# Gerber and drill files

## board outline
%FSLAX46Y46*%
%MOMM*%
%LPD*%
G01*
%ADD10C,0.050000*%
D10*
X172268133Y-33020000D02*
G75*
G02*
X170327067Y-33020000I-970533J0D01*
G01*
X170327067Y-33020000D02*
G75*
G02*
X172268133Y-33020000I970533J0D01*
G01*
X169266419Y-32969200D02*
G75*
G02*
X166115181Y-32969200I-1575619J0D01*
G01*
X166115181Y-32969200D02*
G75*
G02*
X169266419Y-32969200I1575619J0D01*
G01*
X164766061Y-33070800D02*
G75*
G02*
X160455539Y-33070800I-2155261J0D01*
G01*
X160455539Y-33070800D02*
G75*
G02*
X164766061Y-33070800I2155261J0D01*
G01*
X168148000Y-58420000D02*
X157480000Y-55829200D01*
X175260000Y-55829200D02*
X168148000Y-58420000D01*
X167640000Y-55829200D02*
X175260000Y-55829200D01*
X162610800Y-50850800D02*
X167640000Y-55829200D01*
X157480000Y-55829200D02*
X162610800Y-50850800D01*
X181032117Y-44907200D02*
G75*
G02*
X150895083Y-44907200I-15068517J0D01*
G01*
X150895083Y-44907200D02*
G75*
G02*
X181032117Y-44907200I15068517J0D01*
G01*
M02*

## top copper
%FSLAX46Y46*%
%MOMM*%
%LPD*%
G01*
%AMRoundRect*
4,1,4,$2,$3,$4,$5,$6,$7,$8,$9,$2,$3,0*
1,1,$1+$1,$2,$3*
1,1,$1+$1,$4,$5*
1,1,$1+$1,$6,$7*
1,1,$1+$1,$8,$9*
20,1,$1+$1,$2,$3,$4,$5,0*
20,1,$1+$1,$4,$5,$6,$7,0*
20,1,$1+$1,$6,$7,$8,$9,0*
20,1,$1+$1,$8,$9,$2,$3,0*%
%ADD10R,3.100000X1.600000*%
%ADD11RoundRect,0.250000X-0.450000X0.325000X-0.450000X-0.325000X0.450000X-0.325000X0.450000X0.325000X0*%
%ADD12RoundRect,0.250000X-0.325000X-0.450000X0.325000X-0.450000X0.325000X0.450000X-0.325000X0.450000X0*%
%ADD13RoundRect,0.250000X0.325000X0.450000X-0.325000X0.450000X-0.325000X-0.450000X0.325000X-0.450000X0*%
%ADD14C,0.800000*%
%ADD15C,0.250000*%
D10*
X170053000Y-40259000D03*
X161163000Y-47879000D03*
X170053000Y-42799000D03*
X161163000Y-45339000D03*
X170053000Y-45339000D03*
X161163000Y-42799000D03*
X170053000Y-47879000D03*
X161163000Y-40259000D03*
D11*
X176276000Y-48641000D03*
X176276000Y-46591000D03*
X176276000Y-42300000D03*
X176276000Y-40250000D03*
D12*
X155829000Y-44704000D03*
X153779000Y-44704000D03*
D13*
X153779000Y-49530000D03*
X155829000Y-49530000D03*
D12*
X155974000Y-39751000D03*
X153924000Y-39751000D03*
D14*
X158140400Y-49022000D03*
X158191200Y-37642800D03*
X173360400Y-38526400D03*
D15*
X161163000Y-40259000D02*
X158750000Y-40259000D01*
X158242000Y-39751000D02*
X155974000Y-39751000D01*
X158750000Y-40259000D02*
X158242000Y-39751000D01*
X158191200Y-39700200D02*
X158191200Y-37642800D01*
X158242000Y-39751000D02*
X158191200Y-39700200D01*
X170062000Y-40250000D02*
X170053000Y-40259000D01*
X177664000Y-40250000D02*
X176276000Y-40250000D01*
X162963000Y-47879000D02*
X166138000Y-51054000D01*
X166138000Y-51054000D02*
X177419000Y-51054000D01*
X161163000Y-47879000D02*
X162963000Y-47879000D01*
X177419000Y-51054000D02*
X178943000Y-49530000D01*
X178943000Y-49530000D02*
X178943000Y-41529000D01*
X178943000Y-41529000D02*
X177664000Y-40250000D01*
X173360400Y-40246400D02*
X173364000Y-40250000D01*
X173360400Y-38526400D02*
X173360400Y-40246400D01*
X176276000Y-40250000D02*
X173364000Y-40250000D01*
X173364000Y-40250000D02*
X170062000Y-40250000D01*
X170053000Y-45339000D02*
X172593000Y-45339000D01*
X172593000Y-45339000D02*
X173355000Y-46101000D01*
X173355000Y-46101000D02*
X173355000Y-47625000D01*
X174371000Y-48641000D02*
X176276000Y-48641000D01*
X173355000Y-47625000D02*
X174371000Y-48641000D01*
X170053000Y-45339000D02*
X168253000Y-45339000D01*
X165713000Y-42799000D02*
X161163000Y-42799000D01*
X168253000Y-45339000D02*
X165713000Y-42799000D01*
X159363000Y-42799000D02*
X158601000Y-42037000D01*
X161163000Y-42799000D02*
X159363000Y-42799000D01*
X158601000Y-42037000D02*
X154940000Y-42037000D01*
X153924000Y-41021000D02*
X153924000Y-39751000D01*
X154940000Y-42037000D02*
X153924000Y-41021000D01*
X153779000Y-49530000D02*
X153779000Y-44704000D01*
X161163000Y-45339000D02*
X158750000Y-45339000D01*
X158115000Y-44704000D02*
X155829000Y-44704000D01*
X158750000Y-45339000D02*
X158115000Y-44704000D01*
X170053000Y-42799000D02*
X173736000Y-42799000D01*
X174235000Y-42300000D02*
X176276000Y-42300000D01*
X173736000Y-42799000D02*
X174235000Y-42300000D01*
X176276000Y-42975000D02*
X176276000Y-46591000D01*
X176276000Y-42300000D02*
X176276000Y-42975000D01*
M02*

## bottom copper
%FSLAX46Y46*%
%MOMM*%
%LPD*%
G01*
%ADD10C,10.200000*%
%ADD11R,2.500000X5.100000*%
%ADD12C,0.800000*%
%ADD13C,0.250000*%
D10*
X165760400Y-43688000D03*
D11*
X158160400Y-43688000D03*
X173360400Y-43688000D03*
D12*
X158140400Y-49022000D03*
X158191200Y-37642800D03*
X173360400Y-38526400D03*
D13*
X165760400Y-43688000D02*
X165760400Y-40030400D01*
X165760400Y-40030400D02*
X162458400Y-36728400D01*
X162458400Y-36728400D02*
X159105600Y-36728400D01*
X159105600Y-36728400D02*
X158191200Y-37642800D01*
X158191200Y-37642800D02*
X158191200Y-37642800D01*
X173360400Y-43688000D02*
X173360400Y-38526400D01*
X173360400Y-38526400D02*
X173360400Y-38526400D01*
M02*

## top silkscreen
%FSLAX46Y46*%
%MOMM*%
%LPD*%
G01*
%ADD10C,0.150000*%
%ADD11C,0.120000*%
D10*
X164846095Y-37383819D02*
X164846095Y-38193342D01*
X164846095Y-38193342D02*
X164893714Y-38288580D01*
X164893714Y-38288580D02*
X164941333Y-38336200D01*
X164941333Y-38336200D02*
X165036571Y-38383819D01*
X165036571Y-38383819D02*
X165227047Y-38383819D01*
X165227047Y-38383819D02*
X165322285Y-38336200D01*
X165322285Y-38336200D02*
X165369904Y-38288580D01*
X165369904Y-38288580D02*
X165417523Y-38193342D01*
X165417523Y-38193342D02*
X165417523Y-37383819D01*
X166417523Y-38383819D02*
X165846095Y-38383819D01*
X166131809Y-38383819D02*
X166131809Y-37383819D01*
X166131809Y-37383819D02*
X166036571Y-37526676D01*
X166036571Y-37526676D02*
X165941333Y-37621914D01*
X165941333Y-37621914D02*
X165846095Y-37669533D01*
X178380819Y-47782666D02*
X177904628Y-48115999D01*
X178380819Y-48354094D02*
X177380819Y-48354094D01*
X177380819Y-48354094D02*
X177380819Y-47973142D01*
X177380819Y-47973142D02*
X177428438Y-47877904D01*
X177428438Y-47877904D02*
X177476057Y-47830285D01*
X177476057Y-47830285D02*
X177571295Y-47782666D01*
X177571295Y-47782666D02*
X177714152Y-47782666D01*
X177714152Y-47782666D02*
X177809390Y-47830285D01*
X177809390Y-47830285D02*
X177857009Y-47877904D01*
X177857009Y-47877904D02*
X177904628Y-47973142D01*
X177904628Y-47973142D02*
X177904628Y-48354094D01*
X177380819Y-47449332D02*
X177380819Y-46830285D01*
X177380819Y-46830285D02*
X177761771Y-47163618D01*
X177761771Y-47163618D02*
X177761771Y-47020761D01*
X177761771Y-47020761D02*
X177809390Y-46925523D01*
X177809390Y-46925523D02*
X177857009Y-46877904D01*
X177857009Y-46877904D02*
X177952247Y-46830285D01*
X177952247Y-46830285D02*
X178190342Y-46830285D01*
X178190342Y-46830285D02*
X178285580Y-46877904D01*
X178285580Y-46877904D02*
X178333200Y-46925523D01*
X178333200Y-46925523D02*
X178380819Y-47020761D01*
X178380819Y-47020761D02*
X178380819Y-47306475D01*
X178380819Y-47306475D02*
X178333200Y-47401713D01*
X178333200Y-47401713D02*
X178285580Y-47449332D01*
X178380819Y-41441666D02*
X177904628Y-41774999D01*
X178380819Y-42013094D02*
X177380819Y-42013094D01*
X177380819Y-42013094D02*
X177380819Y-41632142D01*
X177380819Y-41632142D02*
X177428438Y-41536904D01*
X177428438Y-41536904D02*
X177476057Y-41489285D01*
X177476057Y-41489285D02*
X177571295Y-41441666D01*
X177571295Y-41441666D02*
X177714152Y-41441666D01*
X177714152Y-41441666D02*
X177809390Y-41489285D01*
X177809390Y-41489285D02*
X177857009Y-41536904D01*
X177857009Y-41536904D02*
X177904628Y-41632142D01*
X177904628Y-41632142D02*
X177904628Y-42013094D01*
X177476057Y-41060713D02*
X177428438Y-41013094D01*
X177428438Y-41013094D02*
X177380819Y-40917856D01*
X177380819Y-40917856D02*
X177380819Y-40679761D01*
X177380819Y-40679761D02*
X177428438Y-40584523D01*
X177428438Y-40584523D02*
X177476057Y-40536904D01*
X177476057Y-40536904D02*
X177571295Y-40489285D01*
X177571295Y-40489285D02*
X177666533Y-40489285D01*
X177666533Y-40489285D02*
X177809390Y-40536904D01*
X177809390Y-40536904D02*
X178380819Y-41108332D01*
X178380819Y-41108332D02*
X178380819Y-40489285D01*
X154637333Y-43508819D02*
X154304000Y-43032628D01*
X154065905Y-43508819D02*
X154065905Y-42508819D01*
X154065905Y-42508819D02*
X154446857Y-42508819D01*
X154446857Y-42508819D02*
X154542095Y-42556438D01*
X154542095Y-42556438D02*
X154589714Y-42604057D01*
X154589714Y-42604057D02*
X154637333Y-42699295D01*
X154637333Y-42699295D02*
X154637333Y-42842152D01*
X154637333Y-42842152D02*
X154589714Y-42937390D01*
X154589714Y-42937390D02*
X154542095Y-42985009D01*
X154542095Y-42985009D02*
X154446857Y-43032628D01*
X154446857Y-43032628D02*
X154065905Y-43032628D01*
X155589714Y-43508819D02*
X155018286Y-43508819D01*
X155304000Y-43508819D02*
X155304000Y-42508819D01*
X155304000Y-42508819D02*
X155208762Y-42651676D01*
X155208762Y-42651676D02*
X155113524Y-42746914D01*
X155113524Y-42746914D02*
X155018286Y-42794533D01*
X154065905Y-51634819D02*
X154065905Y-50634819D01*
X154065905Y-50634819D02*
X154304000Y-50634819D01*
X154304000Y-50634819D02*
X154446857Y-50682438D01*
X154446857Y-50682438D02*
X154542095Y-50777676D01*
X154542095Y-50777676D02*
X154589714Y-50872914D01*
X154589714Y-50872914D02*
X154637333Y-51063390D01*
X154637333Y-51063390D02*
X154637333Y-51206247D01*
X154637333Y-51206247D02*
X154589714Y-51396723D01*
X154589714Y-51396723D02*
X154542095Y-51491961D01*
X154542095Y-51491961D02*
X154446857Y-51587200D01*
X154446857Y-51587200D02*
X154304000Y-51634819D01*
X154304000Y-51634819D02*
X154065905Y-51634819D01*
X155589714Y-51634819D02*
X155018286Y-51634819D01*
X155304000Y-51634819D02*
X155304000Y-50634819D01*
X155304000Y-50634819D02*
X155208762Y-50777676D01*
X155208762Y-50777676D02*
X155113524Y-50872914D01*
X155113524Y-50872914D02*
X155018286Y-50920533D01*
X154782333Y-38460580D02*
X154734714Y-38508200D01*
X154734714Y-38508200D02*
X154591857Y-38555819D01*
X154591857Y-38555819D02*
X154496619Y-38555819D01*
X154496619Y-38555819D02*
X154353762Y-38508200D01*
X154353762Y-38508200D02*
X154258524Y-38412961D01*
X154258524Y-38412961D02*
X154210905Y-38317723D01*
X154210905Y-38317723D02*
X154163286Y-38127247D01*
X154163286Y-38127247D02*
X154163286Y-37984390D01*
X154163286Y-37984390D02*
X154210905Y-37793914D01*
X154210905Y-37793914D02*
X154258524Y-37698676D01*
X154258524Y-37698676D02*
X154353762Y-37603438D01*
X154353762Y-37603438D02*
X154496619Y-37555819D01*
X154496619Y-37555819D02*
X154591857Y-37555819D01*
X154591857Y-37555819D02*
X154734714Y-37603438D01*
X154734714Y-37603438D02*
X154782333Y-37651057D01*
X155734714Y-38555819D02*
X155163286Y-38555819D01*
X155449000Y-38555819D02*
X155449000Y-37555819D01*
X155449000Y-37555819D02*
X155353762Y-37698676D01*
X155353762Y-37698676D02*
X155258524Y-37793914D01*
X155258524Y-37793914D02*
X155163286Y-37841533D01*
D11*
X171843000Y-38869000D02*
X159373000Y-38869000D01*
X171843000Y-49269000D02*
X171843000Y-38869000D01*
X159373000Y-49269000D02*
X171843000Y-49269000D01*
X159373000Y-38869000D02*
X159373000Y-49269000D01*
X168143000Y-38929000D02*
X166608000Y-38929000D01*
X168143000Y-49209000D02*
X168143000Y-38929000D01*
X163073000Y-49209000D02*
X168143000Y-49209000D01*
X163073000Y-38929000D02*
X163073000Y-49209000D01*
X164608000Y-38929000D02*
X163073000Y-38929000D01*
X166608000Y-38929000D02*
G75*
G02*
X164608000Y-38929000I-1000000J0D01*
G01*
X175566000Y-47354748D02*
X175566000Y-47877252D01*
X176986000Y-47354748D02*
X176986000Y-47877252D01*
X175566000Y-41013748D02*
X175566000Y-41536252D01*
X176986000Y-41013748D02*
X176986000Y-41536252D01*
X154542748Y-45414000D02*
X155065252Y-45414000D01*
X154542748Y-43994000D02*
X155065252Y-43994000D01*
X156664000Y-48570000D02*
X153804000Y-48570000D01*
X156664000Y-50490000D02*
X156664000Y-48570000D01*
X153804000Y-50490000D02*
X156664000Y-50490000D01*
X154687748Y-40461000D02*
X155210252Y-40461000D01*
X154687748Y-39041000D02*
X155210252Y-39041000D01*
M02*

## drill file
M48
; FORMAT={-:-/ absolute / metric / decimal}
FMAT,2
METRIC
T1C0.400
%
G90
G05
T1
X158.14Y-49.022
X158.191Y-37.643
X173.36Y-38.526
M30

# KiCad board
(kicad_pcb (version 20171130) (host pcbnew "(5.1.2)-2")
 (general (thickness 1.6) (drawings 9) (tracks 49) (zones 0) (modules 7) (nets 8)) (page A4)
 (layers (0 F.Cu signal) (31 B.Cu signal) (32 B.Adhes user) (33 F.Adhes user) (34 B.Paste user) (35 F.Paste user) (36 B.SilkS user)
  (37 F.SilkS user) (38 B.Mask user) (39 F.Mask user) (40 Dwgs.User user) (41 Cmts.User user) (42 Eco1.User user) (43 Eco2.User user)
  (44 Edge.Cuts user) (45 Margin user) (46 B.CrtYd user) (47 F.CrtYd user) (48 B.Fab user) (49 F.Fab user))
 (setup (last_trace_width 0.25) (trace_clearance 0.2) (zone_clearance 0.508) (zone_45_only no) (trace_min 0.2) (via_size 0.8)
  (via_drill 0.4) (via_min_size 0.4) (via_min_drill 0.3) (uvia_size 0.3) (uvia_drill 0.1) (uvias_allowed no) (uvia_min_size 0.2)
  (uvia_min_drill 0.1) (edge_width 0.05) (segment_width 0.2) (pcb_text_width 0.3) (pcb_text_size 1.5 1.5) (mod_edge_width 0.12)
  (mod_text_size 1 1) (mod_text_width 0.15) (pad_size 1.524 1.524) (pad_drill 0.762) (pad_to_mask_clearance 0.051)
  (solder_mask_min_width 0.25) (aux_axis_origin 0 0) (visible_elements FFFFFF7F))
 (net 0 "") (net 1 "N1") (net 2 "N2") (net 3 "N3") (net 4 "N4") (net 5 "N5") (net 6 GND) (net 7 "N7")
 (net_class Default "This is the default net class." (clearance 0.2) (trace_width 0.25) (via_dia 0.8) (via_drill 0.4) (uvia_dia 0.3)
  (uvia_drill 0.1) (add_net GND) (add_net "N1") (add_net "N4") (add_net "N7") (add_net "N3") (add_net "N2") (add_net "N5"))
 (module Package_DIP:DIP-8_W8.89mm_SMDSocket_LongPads (layer F.Cu) (at 165.608 44.069)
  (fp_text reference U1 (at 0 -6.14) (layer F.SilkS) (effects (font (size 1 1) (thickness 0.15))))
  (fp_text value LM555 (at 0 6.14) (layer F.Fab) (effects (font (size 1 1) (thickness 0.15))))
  (fp_line (start 6.235 -5.2) (end -6.235 -5.2) (layer F.SilkS) (width 0.12))
  (fp_line (start 6.235 5.2) (end 6.235 -5.2) (layer F.SilkS) (width 0.12))
  (fp_line (start -6.235 5.2) (end 6.235 5.2) (layer F.SilkS) (width 0.12))
  (fp_line (start -6.235 -5.2) (end -6.235 5.2) (layer F.SilkS) (width 0.12))
  (fp_line (start 2.535 -5.14) (end 1 -5.14) (layer F.SilkS) (width 0.12))
  (fp_line (start 2.535 5.14) (end 2.535 -5.14) (layer F.SilkS) (width 0.12))
  (fp_line (start -2.535 5.14) (end 2.535 5.14) (layer F.SilkS) (width 0.12))
  (fp_line (start -2.535 -5.14) (end -2.535 5.14) (layer F.SilkS) (width 0.12))
  (fp_line (start -1 -5.14) (end -2.535 -5.14) (layer F.SilkS) (width 0.12))
  (fp_arc (start 0 -5.14) (end -1 -5.14) (angle -180) (layer F.SilkS) (width 0.12))
  (pad 8 smd rect (at 4.445 -3.81) (size 3.1 1.6) (layers F.Cu F.Paste F.Mask) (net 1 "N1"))
  (pad 4 smd rect (at -4.445 3.81) (size 3.1 1.6) (layers F.Cu F.Paste F.Mask) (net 1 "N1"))
  (pad 7 smd rect (at 4.445 -1.27) (size 3.1 1.6) (layers F.Cu F.Paste F.Mask) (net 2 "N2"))
  (pad 3 smd rect (at -4.445 1.27) (size 3.1 1.6) (layers F.Cu F.Paste F.Mask) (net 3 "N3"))
  (pad 6 smd rect (at 4.445 1.27) (size 3.1 1.6) (layers F.Cu F.Paste F.Mask) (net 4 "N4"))
  (pad 2 smd rect (at -4.445 -1.27) (size 3.1 1.6) (layers F.Cu F.Paste F.Mask) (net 4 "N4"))
  (pad 5 smd rect (at 4.445 3.81) (size 3.1 1.6) (layers F.Cu F.Paste F.Mask) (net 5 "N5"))
  (pad 1 smd rect (at -4.445 -3.81) (size 3.1 1.6) (layers F.Cu F.Paste F.Mask) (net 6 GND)))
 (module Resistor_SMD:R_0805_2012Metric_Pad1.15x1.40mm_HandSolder (layer F.Cu) (at 176.276 47.616 270)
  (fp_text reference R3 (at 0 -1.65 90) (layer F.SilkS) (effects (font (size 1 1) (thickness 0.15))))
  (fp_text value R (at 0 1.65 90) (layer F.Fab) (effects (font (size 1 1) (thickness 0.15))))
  (fp_line (start -0.261252 0.71) (end 0.261252 0.71) (layer F.SilkS) (width 0.12))
  (fp_line (start -0.261252 -0.71) (end 0.261252 -0.71) (layer F.SilkS) (width 0.12))
  (pad 2 smd roundrect (at 1.025 0 270) (size 1.15 1.4) (layers F.Cu F.Paste F.Mask) (roundrect_rratio 0.217391) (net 4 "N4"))
  (pad 1 smd roundrect (at -1.025 0 270) (size 1.15 1.4) (layers F.Cu F.Paste F.Mask) (roundrect_rratio 0.217391) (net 2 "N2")))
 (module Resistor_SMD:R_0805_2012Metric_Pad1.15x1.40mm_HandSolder (layer F.Cu) (at 176.276 41.275 270)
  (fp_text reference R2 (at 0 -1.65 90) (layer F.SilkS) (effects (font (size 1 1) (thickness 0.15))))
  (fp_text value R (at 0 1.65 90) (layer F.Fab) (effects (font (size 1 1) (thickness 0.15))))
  (fp_line (start -0.261252 0.71) (end 0.261252 0.71) (layer F.SilkS) (width 0.12))
  (fp_line (start -0.261252 -0.71) (end 0.261252 -0.71) (layer F.SilkS) (width 0.12))
  (pad 2 smd roundrect (at 1.025 0 270) (size 1.15 1.4) (layers F.Cu F.Paste F.Mask) (roundrect_rratio 0.217391) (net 2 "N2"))
  (pad 1 smd roundrect (at -1.025 0 270) (size 1.15 1.4) (layers F.Cu F.Paste F.Mask) (roundrect_rratio 0.217391) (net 1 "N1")))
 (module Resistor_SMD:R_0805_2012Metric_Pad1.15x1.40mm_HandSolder (layer F.Cu) (at 154.804 44.704)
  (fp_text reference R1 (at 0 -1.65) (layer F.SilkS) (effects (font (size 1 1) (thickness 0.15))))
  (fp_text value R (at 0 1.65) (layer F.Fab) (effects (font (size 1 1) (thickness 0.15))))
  (fp_line (start -0.261252 0.71) (end 0.261252 0.71) (layer F.SilkS) (width 0.12))
  (fp_line (start -0.261252 -0.71) (end 0.261252 -0.71) (layer F.SilkS) (width 0.12))
  (pad 2 smd roundrect (at 1.025 0) (size 1.15 1.4) (layers F.Cu F.Paste F.Mask) (roundrect_rratio 0.217391) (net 3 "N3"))
  (pad 1 smd roundrect (at -1.025 0) (size 1.15 1.4) (layers F.Cu F.Paste F.Mask) (roundrect_rratio 0.217391) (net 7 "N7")))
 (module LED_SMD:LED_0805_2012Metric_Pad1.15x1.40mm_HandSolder (layer F.Cu) (at 154.804 49.53 180)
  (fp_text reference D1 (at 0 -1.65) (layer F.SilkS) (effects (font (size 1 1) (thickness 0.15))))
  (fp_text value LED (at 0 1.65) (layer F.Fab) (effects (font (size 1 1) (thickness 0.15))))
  (fp_line (start -1.86 0.96) (end 1 0.96) (layer F.SilkS) (width 0.12))
  (fp_line (start -1.86 -0.96) (end -1.86 0.96) (layer F.SilkS) (width 0.12))
  (fp_line (start 1 -0.96) (end -1.86 -0.96) (layer F.SilkS) (width 0.12))
  (pad 2 smd roundrect (at 1.025 0 180) (size 1.15 1.4) (layers F.Cu F.Paste F.Mask) (roundrect_rratio 0.217391) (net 7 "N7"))
  (pad 1 smd roundrect (at -1.025 0 180) (size 1.15 1.4) (layers F.Cu F.Paste F.Mask) (roundrect_rratio 0.217391) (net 6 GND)))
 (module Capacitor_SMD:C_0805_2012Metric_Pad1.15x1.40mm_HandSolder (layer F.Cu) (at 154.949 39.751)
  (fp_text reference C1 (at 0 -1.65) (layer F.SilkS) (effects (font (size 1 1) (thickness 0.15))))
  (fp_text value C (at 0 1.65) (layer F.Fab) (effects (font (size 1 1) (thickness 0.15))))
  (fp_line (start -0.261252 0.71) (end 0.261252 0.71) (layer F.SilkS) (width 0.12))
  (fp_line (start -0.261252 -0.71) (end 0.261252 -0.71) (layer F.SilkS) (width 0.12))
  (pad 2 smd roundrect (at 1.025 0) (size 1.15 1.4) (layers F.Cu F.Paste F.Mask) (roundrect_rratio 0.217391) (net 6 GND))
  (pad 1 smd roundrect (at -1.025 0) (size 1.15 1.4) (layers F.Cu F.Paste F.Mask) (roundrect_rratio 0.217391) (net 4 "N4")))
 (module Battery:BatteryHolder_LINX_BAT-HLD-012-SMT (layer B.Cu) (at 165.7604 43.688 180)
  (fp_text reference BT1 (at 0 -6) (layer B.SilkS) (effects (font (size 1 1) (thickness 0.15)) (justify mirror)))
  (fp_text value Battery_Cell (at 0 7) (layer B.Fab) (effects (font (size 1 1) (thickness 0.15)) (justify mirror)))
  (pad 2 smd circle (at 0 0 180) (size 10.2 10.2) (layers B.Cu B.Paste B.Mask) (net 6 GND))
  (pad 1 smd rect (at 7.6 0 180) (size 2.5 5.1) (layers B.Cu B.Paste B.Mask) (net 1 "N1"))
  (pad 1 smd rect (at -7.6 0 180) (size 2.5 5.1) (layers B.Cu B.Paste B.Mask) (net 1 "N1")))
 (gr_circle (center 171.2976 33.02) (end 172.2628 32.9184) (layer Edge.Cuts) (width 0.05))
 (gr_circle (center 167.6908 32.9692) (end 169.2656 33.02) (layer Edge.Cuts) (width 0.05))
 (gr_circle (center 162.6108 33.0708) (end 164.7444 32.766) (layer Edge.Cuts) (width 0.05))
 (gr_line (start 168.148 58.42) (end 157.48 55.8292) (layer Edge.Cuts) (width 0.05))
 (gr_line (start 175.26 55.8292) (end 168.148 58.42) (layer Edge.Cuts) (width 0.05))
 (gr_line (start 167.64 55.8292) (end 175.26 55.8292) (layer Edge.Cuts) (width 0.05))
 (gr_line (start 162.6108 50.8508) (end 167.64 55.8292) (layer Edge.Cuts) (width 0.05))
 (gr_line (start 157.48 55.8292) (end 162.6108 50.8508) (layer Edge.Cuts) (width 0.05))
 (gr_circle (center 165.9636 44.9072) (end 152.2984 38.5572) (layer Edge.Cuts) (width 0.05))
 (via (at 158.1404 49.022) (size 0.8) (drill 0.4) (layers F.Cu B.Cu) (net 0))
 (segment (start 161.163 40.259) (end 158.75 40.259) (width 0.25) (layer F.Cu) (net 6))
 (segment (start 158.242 39.751) (end 155.974 39.751) (width 0.25) (layer F.Cu) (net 6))
 (segment (start 158.75 40.259) (end 158.242 39.751) (width 0.25) (layer F.Cu) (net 6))
 (segment (start 165.7604 43.688) (end 165.7604 40.0304) (width 0.25) (layer B.Cu) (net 6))
 (segment (start 165.7604 40.0304) (end 162.4584 36.7284) (width 0.25) (layer B.Cu) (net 6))
 (segment (start 162.4584 36.7284) (end 159.1056 36.7284) (width 0.25) (layer B.Cu) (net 6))
 (segment (start 159.1056 36.7284) (end 158.1912 37.6428) (width 0.25) (layer B.Cu) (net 6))
 (segment (start 158.1912 37.6428) (end 158.1912 37.6428) (width 0.25) (layer B.Cu) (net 6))
 (via (at 158.1912 37.6428) (size 0.8) (drill 0.4) (layers F.Cu B.Cu) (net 6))
 (segment (start 158.1912 39.7002) (end 158.1912 37.6428) (width 0.25) (layer F.Cu) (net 6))
 (segment (start 158.242 39.751) (end 158.1912 39.7002) (width 0.25) (layer F.Cu) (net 6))
 (segment (start 170.062 40.25) (end 170.053 40.259) (width 0.25) (layer F.Cu) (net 1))
 (segment (start 177.664 40.25) (end 176.276 40.25) (width 0.25) (layer F.Cu) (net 1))
 (segment (start 162.963 47.879) (end 166.138 51.054) (width 0.25) (layer F.Cu) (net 1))
 (segment (start 166.138 51.054) (end 177.419 51.054) (width 0.25) (layer F.Cu) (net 1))
 (segment (start 161.163 47.879) (end 162.963 47.879) (width 0.25) (layer F.Cu) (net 1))
 (segment (start 177.419 51.054) (end 178.943 49.53) (width 0.25) (layer F.Cu) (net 1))
 (segment (start 178.943 49.53) (end 178.943 41.529) (width 0.25) (layer F.Cu) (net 1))
 (segment (start 178.943 41.529) (end 177.664 40.25) (width 0.25) (layer F.Cu) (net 1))
 (segment (start 173.3604 43.688) (end 173.3604 38.5264) (width 0.25) (layer B.Cu) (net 1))
 (segment (start 173.3604 38.5264) (end 173.3604 38.5264) (width 0.25) (layer B.Cu) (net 1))
 (via (at 173.3604 38.5264) (size 0.8) (drill 0.4) (layers F.Cu B.Cu) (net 1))
 (segment (start 173.3604 40.2464) (end 173.364 40.25) (width 0.25) (layer F.Cu) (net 1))
 (segment (start 173.3604 38.5264) (end 173.3604 40.2464) (width 0.25) (layer F.Cu) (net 1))
 (segment (start 176.276 40.25) (end 173.364 40.25) (width 0.25) (layer F.Cu) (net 1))
 (segment (start 173.364 40.25) (end 170.062 40.25) (width 0.25) (layer F.Cu) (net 1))
 (segment (start 170.053 45.339) (end 172.593 45.339) (width 0.25) (layer F.Cu) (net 4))
 (segment (start 172.593 45.339) (end 173.355 46.101) (width 0.25) (layer F.Cu) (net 4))
 (segment (start 173.355 46.101) (end 173.355 47.625) (width 0.25) (layer F.Cu) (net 4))
 (segment (start 174.371 48.641) (end 176.276 48.641) (width 0.25) (layer F.Cu) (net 4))
 (segment (start 173.355 47.625) (end 174.371 48.641) (width 0.25) (layer F.Cu) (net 4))
 (segment (start 170.053 45.339) (end 168.253 45.339) (width 0.25) (layer F.Cu) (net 4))
 (segment (start 165.713 42.799) (end 161.163 42.799) (width 0.25) (layer F.Cu) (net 4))
 (segment (start 168.253 45.339) (end 165.713 42.799) (width 0.25) (layer F.Cu) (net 4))
 (segment (start 159.363 42.799) (end 158.601 42.037) (width 0.25) (layer F.Cu) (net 4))
 (segment (start 161.163 42.799) (end 159.363 42.799) (width 0.25) (layer F.Cu) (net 4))
 (segment (start 158.601 42.037) (end 154.94 42.037) (width 0.25) (layer F.Cu) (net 4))
 (segment (start 153.924 41.021) (end 153.924 39.751) (width 0.25) (layer F.Cu) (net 4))
 (segment (start 154.94 42.037) (end 153.924 41.021) (width 0.25) (layer F.Cu) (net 4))
 (segment (start 153.779 49.53) (end 153.779 44.704) (width 0.25) (layer F.Cu) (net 7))
 (segment (start 161.163 45.339) (end 158.75 45.339) (width 0.25) (layer F.Cu) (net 3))
 (segment (start 158.115 44.704) (end 155.829 44.704) (width 0.25) (layer F.Cu) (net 3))
 (segment (start 158.75 45.339) (end 158.115 44.704) (width 0.25) (layer F.Cu) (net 3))
 (segment (start 170.053 42.799) (end 173.736 42.799) (width 0.25) (layer F.Cu) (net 2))
 (segment (start 174.235 42.3) (end 176.276 42.3) (width 0.25) (layer F.Cu) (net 2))
 (segment (start 173.736 42.799) (end 174.235 42.3) (width 0.25) (layer F.Cu) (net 2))
 (segment (start 176.276 42.975) (end 176.276 46.591) (width 0.25) (layer F.Cu) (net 2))
 (segment (start 176.276 42.3) (end 176.276 42.975) (width 0.25) (layer F.Cu) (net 2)))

